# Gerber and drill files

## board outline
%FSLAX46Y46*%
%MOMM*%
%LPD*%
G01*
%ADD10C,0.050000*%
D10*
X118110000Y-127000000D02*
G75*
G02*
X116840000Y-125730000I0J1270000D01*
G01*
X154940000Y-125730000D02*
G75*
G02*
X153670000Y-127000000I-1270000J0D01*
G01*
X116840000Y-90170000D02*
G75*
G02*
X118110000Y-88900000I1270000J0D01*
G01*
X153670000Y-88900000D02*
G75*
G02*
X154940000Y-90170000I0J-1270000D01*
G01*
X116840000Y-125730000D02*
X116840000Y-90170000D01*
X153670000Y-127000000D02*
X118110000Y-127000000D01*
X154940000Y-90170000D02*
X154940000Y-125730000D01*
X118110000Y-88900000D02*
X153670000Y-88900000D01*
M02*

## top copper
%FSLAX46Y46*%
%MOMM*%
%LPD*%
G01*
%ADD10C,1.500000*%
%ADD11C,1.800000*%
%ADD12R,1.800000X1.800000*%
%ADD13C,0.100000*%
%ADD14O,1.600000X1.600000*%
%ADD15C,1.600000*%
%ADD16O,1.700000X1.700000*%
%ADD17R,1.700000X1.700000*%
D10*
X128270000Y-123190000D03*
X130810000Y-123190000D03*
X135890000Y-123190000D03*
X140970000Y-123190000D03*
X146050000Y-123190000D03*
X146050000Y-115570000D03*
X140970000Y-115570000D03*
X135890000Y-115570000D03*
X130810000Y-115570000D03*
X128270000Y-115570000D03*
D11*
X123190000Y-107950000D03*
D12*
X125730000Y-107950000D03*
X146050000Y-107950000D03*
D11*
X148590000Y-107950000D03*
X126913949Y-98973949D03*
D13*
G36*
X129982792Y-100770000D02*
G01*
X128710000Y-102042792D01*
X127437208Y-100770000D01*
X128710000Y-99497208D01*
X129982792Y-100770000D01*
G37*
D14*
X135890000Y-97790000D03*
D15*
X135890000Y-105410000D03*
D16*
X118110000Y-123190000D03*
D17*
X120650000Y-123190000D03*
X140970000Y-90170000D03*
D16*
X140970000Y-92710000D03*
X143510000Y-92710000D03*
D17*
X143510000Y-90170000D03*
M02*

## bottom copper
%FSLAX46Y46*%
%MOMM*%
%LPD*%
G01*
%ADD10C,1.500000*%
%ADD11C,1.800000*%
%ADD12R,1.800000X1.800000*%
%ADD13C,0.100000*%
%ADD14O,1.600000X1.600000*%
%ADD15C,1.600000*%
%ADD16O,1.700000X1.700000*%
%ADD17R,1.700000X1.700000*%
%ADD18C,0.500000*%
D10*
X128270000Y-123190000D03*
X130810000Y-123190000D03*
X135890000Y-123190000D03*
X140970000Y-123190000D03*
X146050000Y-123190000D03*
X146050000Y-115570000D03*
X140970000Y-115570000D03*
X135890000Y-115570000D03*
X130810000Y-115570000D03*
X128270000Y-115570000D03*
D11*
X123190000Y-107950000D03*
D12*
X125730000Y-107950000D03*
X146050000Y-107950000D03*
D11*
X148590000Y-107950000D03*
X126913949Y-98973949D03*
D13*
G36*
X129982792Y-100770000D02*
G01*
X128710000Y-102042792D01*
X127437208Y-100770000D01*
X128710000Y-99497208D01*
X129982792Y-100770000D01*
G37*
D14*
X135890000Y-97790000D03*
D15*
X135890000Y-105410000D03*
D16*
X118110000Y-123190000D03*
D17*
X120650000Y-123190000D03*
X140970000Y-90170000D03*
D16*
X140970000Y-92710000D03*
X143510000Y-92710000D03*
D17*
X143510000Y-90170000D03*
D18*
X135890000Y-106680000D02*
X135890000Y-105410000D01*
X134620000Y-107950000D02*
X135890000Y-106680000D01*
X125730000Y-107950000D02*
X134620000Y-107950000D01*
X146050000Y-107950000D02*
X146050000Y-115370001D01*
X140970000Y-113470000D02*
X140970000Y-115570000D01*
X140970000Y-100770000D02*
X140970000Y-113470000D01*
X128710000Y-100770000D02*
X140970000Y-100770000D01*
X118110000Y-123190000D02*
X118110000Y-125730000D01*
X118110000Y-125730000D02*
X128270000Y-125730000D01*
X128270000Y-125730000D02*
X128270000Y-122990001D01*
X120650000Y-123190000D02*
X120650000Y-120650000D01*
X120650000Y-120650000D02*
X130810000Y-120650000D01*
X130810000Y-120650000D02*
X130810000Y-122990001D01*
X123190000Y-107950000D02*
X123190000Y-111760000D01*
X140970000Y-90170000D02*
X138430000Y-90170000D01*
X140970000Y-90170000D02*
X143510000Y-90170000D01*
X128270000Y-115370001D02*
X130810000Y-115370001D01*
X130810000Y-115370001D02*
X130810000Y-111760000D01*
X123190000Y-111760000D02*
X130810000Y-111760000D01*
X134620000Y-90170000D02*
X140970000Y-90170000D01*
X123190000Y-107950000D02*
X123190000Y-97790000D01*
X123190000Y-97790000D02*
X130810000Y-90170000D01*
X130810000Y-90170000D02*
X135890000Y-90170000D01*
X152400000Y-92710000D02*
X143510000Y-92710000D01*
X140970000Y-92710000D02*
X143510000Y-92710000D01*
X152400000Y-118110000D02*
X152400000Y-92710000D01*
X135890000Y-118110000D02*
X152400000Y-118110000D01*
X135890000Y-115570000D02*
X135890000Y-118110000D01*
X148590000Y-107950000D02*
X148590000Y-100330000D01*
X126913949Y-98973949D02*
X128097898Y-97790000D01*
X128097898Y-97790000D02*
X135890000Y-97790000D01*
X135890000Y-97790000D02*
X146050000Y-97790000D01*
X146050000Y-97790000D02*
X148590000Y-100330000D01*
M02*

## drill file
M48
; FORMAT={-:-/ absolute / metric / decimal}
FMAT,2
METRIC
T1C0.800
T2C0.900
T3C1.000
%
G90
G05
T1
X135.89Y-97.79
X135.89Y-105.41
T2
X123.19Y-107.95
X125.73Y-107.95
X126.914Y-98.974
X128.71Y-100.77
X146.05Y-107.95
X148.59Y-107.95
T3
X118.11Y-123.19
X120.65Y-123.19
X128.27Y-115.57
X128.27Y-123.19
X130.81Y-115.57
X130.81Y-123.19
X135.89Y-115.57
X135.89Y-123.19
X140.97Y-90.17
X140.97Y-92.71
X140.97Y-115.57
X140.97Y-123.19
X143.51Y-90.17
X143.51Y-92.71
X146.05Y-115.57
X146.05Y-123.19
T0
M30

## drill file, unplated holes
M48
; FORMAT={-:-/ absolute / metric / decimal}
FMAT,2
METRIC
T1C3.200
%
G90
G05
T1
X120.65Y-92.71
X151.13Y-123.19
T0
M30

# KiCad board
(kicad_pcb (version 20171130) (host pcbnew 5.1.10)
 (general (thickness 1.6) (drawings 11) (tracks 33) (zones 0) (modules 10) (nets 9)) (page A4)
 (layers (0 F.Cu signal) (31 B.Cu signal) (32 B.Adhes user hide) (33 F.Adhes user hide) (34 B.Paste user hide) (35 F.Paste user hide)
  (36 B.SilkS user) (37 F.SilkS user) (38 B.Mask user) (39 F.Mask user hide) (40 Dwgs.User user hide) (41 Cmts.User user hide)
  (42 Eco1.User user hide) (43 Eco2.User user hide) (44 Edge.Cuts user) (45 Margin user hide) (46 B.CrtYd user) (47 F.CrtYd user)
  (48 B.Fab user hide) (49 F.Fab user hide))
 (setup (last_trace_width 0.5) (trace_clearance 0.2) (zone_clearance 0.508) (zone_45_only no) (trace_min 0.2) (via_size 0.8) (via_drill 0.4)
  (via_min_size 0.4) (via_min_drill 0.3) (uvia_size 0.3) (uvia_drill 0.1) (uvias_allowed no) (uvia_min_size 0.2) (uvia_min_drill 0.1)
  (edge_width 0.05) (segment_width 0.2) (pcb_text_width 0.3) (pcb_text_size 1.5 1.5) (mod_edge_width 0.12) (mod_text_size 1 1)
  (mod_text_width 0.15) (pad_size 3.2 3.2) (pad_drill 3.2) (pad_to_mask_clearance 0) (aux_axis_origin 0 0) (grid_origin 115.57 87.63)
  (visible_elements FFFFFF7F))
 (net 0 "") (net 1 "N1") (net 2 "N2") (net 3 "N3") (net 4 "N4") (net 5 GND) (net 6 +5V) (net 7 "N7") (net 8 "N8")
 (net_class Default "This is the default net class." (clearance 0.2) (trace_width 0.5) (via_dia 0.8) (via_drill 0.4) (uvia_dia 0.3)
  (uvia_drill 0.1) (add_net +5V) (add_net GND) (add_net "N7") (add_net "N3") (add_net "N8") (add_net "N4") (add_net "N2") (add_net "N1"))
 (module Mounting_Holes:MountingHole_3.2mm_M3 (layer F.Cu) (at 120.65 92.71)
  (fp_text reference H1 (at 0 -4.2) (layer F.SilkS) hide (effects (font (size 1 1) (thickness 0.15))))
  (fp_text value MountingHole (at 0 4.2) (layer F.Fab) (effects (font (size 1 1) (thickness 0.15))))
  (pad "" np_thru_hole circle (at 0 0) (size 3.2 3.2) (drill 3.2) (layers *.Cu *.Mask) (thermal_gap 2)))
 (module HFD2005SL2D (layer F.Cu) (at 128.27 123.19)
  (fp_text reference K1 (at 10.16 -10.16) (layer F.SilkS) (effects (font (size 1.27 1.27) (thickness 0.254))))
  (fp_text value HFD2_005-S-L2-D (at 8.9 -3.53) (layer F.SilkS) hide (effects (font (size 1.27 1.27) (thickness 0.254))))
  (pad 1 thru_hole circle (at 0 0 90) (size 1.5 1.5) (drill 1) (layers *.Cu *.Mask F.SilkS) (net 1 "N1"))
  (pad 2 thru_hole circle (at 2.54 0 90) (size 1.5 1.5) (drill 1) (layers *.Cu *.Mask F.SilkS) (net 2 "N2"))
  (pad 4 thru_hole circle (at 7.62 0 90) (size 1.5 1.5) (drill 1) (layers *.Cu *.Mask F.SilkS))
  (pad 6 thru_hole circle (at 12.7 0 90) (size 1.5 1.5) (drill 1) (layers *.Cu *.Mask F.SilkS))
  (pad 8 thru_hole circle (at 17.78 0 90) (size 1.5 1.5) (drill 1) (layers *.Cu *.Mask F.SilkS))
  (pad 9 thru_hole circle (at 17.78 -7.62 90) (size 1.5 1.5) (drill 1) (layers *.Cu *.Mask F.SilkS) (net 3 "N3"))
  (pad 11 thru_hole circle (at 12.7 -7.62 90) (size 1.5 1.5) (drill 1) (layers *.Cu *.Mask F.SilkS) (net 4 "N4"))
  (pad 13 thru_hole circle (at 7.62 -7.62 90) (size 1.5 1.5) (drill 1) (layers *.Cu *.Mask F.SilkS) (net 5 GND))
  (pad 15 thru_hole circle (at 2.54 -7.62 90) (size 1.5 1.5) (drill 1) (layers *.Cu *.Mask F.SilkS) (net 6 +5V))
  (pad 16 thru_hole circle (at 0 -7.62 90) (size 1.5 1.5) (drill 1) (layers *.Cu *.Mask F.SilkS) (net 6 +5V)))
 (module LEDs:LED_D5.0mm (layer F.Cu) (at 125.73 107.95 180)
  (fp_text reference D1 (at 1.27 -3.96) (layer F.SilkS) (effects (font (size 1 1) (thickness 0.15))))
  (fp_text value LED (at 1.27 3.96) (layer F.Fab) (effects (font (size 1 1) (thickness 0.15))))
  (pad 2 thru_hole circle (at 2.54 0 180) (size 1.8 1.8) (drill 0.9) (layers *.Cu *.Mask) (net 6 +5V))
  (pad 1 thru_hole rect (at 0 0 180) (size 1.8 1.8) (drill 0.9) (layers *.Cu *.Mask) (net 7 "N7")))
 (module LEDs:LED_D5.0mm (layer F.Cu) (at 146.05 107.95)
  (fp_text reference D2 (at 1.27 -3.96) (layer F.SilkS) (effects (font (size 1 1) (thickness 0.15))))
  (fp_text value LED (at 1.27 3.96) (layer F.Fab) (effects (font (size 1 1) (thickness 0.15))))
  (pad 1 thru_hole rect (at 0 0) (size 1.8 1.8) (drill 0.9) (layers *.Cu *.Mask) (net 3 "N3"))
  (pad 2 thru_hole circle (at 2.54 0) (size 1.8 1.8) (drill 0.9) (layers *.Cu *.Mask) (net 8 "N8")))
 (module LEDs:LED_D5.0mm (layer F.Cu) (at 128.71 100.77 135)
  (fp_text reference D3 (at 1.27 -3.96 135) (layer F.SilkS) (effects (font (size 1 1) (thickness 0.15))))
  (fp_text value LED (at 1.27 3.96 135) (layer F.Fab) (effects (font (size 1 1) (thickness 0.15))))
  (pad 2 thru_hole circle (at 2.54 0 135) (size 1.8 1.8) (drill 0.9) (layers *.Cu *.Mask) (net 8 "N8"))
  (pad 1 thru_hole rect (at 0 0 135) (size 1.8 1.8) (drill 0.9) (layers *.Cu *.Mask) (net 4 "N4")))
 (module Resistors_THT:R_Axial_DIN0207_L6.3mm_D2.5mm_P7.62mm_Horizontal (layer F.Cu) (at 135.89 105.41 90)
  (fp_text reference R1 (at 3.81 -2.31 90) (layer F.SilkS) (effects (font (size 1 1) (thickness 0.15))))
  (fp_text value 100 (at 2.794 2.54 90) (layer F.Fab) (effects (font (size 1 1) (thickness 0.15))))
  (pad 2 thru_hole oval (at 7.62 0 90) (size 1.6 1.6) (drill 0.8) (layers *.Cu *.Mask) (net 8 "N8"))
  (pad 1 thru_hole circle (at 0 0 90) (size 1.6 1.6) (drill 0.8) (layers *.Cu *.Mask) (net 7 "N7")))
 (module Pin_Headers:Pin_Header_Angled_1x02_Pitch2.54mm (layer B.Cu) (at 120.65 123.19 90)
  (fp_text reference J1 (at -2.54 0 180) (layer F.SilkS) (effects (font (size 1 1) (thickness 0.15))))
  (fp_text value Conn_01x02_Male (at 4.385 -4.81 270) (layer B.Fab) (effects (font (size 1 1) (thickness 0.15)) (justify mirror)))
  (pad 2 thru_hole oval (at 0 -2.54 90) (size 1.7 1.7) (drill 1) (layers *.Cu *.Mask) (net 1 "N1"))
  (pad 1 thru_hole rect (at 0 0 90) (size 1.7 1.7) (drill 1) (layers *.Cu *.Mask) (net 2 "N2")))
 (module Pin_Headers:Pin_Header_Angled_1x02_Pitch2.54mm (layer B.Cu) (at 140.97 90.17 180)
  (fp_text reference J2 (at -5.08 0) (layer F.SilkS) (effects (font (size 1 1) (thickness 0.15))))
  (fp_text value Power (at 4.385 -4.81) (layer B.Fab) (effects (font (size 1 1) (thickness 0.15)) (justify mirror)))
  (pad 1 thru_hole rect (at 0 0 180) (size 1.7 1.7) (drill 1) (layers *.Cu *.Mask) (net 6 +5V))
  (pad 2 thru_hole oval (at 0 -2.54 180) (size 1.7 1.7) (drill 1) (layers *.Cu *.Mask) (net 5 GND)))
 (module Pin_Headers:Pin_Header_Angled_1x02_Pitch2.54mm (layer B.Cu) (at 143.51 90.17 180)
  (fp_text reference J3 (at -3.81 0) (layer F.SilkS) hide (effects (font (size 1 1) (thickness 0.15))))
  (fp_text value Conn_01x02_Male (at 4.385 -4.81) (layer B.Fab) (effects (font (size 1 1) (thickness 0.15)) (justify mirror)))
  (pad 2 thru_hole oval (at 0 -2.54 180) (size 1.7 1.7) (drill 1) (layers *.Cu *.Mask) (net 5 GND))
  (pad 1 thru_hole rect (at 0 0 180) (size 1.7 1.7) (drill 1) (layers *.Cu *.Mask) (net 6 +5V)))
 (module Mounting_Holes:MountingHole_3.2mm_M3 (layer F.Cu) (at 151.13 123.19)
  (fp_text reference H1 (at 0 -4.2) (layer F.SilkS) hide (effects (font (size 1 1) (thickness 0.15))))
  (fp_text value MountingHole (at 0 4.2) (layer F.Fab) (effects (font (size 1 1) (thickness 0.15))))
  (pad "" np_thru_hole circle (at 0 0) (size 3.2 3.2) (drill 3.2) (layers *.Cu *.Mask) (thermal_gap 2)))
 (gr_arc (start 118.11 125.73) (end 116.84 125.73) (angle -90) (layer Edge.Cuts) (width 0.05))
 (gr_arc (start 153.67 125.73) (end 153.67 127) (angle -90) (layer Edge.Cuts) (width 0.05))
 (gr_arc (start 118.11 90.17) (end 118.11 88.9) (angle -90) (layer Edge.Cuts) (width 0.05))
 (gr_arc (start 153.67 90.17) (end 154.94 90.17) (angle -90) (layer Edge.Cuts) (width 0.05))
 (gr_line (start 116.84 125.73) (end 116.84 90.17) (layer Edge.Cuts) (width 0.05))
 (gr_line (start 153.67 127) (end 118.11 127) (layer Edge.Cuts) (width 0.05))
 (gr_line (start 154.94 90.17) (end 154.94 125.73) (layer Edge.Cuts) (width 0.05))
 (gr_line (start 118.11 88.9) (end 153.67 88.9) (layer Edge.Cuts) (width 0.05))
 (segment (start 135.89 106.68) (end 135.89 105.41) (width 0.5) (layer B.Cu) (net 7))
 (segment (start 134.62 107.95) (end 135.89 106.68) (width 0.5) (layer B.Cu) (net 7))
 (segment (start 125.73 107.95) (end 134.62 107.95) (width 0.5) (layer B.Cu) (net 7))
 (segment (start 146.05 107.95) (end 146.05 115.370001) (width 0.5) (layer B.Cu) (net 3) (status 30))
 (segment (start 140.97 113.47) (end 140.97 115.57) (width 0.5) (layer B.Cu) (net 4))
 (segment (start 140.97 100.77) (end 140.97 113.47) (width 0.5) (layer B.Cu) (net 4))
 (segment (start 128.71 100.77) (end 140.97 100.77) (width 0.5) (layer B.Cu) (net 4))
 (segment (start 118.11 123.19) (end 118.11 125.73) (width 0.5) (layer B.Cu) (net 1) (status 10))
 (segment (start 118.11 125.73) (end 128.27 125.73) (width 0.5) (layer B.Cu) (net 1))
 (segment (start 128.27 125.73) (end 128.27 122.990001) (width 0.5) (layer B.Cu) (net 1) (status 20))
 (segment (start 120.65 123.19) (end 120.65 120.65) (width 0.5) (layer B.Cu) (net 2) (status 10))
 (segment (start 120.65 120.65) (end 130.81 120.65) (width 0.5) (layer B.Cu) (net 2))
 (segment (start 130.81 120.65) (end 130.81 122.990001) (width 0.5) (layer B.Cu) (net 2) (status 20))
 (segment (start 123.19 107.95) (end 123.19 111.76) (width 0.5) (layer B.Cu) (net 6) (status 10))
 (segment (start 140.97 90.17) (end 138.43 90.17) (width 0.5) (layer B.Cu) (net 6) (status 10))
 (segment (start 140.97 90.17) (end 143.51 90.17) (width 0.5) (layer B.Cu) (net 6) (status 30))
 (segment (start 128.27 115.370001) (end 130.81 115.370001) (width 0.5) (layer B.Cu) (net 6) (status 30))
 (segment (start 130.81 115.370001) (end 130.81 111.76) (width 0.5) (layer B.Cu) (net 6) (status 10))
 (segment (start 123.19 111.76) (end 130.81 111.76) (width 0.5) (layer B.Cu) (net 6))
 (segment (start 134.62 90.17) (end 140.97 90.17) (width 0.5) (layer B.Cu) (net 6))
 (segment (start 123.19 107.95) (end 123.19 97.79) (width 0.5) (layer B.Cu) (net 6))
 (segment (start 123.19 97.79) (end 130.81 90.17) (width 0.5) (layer B.Cu) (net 6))
 (segment (start 130.81 90.17) (end 135.89 90.17) (width 0.5) (layer B.Cu) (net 6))
 (segment (start 152.4 92.71) (end 143.51 92.71) (width 0.5) (layer B.Cu) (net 5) (status 20))
 (segment (start 140.97 92.71) (end 143.51 92.71) (width 0.5) (layer B.Cu) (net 5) (status 30))
 (segment (start 152.4 118.11) (end 152.4 92.71) (width 0.5) (layer B.Cu) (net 5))
 (segment (start 135.89 118.11) (end 152.4 118.11) (width 0.5) (layer B.Cu) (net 5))
 (segment (start 135.89 115.57) (end 135.89 118.11) (width 0.5) (layer B.Cu) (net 5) (status 10))
 (segment (start 148.59 107.95) (end 148.59 100.33) (width 0.5) (layer B.Cu) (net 8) (status 10))
 (segment (start 126.913949 98.973949) (end 128.097898 97.79) (width 0.5) (layer B.Cu) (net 8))
 (segment (start 128.097898 97.79) (end 135.89 97.79) (width 0.5) (layer B.Cu) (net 8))
 (segment (start 135.89 97.79) (end 146.05 97.79) (width 0.5) (layer B.Cu) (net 8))
 (segment (start 146.05 97.79) (end 148.59 100.33) (width 0.5) (layer B.Cu) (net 8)))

